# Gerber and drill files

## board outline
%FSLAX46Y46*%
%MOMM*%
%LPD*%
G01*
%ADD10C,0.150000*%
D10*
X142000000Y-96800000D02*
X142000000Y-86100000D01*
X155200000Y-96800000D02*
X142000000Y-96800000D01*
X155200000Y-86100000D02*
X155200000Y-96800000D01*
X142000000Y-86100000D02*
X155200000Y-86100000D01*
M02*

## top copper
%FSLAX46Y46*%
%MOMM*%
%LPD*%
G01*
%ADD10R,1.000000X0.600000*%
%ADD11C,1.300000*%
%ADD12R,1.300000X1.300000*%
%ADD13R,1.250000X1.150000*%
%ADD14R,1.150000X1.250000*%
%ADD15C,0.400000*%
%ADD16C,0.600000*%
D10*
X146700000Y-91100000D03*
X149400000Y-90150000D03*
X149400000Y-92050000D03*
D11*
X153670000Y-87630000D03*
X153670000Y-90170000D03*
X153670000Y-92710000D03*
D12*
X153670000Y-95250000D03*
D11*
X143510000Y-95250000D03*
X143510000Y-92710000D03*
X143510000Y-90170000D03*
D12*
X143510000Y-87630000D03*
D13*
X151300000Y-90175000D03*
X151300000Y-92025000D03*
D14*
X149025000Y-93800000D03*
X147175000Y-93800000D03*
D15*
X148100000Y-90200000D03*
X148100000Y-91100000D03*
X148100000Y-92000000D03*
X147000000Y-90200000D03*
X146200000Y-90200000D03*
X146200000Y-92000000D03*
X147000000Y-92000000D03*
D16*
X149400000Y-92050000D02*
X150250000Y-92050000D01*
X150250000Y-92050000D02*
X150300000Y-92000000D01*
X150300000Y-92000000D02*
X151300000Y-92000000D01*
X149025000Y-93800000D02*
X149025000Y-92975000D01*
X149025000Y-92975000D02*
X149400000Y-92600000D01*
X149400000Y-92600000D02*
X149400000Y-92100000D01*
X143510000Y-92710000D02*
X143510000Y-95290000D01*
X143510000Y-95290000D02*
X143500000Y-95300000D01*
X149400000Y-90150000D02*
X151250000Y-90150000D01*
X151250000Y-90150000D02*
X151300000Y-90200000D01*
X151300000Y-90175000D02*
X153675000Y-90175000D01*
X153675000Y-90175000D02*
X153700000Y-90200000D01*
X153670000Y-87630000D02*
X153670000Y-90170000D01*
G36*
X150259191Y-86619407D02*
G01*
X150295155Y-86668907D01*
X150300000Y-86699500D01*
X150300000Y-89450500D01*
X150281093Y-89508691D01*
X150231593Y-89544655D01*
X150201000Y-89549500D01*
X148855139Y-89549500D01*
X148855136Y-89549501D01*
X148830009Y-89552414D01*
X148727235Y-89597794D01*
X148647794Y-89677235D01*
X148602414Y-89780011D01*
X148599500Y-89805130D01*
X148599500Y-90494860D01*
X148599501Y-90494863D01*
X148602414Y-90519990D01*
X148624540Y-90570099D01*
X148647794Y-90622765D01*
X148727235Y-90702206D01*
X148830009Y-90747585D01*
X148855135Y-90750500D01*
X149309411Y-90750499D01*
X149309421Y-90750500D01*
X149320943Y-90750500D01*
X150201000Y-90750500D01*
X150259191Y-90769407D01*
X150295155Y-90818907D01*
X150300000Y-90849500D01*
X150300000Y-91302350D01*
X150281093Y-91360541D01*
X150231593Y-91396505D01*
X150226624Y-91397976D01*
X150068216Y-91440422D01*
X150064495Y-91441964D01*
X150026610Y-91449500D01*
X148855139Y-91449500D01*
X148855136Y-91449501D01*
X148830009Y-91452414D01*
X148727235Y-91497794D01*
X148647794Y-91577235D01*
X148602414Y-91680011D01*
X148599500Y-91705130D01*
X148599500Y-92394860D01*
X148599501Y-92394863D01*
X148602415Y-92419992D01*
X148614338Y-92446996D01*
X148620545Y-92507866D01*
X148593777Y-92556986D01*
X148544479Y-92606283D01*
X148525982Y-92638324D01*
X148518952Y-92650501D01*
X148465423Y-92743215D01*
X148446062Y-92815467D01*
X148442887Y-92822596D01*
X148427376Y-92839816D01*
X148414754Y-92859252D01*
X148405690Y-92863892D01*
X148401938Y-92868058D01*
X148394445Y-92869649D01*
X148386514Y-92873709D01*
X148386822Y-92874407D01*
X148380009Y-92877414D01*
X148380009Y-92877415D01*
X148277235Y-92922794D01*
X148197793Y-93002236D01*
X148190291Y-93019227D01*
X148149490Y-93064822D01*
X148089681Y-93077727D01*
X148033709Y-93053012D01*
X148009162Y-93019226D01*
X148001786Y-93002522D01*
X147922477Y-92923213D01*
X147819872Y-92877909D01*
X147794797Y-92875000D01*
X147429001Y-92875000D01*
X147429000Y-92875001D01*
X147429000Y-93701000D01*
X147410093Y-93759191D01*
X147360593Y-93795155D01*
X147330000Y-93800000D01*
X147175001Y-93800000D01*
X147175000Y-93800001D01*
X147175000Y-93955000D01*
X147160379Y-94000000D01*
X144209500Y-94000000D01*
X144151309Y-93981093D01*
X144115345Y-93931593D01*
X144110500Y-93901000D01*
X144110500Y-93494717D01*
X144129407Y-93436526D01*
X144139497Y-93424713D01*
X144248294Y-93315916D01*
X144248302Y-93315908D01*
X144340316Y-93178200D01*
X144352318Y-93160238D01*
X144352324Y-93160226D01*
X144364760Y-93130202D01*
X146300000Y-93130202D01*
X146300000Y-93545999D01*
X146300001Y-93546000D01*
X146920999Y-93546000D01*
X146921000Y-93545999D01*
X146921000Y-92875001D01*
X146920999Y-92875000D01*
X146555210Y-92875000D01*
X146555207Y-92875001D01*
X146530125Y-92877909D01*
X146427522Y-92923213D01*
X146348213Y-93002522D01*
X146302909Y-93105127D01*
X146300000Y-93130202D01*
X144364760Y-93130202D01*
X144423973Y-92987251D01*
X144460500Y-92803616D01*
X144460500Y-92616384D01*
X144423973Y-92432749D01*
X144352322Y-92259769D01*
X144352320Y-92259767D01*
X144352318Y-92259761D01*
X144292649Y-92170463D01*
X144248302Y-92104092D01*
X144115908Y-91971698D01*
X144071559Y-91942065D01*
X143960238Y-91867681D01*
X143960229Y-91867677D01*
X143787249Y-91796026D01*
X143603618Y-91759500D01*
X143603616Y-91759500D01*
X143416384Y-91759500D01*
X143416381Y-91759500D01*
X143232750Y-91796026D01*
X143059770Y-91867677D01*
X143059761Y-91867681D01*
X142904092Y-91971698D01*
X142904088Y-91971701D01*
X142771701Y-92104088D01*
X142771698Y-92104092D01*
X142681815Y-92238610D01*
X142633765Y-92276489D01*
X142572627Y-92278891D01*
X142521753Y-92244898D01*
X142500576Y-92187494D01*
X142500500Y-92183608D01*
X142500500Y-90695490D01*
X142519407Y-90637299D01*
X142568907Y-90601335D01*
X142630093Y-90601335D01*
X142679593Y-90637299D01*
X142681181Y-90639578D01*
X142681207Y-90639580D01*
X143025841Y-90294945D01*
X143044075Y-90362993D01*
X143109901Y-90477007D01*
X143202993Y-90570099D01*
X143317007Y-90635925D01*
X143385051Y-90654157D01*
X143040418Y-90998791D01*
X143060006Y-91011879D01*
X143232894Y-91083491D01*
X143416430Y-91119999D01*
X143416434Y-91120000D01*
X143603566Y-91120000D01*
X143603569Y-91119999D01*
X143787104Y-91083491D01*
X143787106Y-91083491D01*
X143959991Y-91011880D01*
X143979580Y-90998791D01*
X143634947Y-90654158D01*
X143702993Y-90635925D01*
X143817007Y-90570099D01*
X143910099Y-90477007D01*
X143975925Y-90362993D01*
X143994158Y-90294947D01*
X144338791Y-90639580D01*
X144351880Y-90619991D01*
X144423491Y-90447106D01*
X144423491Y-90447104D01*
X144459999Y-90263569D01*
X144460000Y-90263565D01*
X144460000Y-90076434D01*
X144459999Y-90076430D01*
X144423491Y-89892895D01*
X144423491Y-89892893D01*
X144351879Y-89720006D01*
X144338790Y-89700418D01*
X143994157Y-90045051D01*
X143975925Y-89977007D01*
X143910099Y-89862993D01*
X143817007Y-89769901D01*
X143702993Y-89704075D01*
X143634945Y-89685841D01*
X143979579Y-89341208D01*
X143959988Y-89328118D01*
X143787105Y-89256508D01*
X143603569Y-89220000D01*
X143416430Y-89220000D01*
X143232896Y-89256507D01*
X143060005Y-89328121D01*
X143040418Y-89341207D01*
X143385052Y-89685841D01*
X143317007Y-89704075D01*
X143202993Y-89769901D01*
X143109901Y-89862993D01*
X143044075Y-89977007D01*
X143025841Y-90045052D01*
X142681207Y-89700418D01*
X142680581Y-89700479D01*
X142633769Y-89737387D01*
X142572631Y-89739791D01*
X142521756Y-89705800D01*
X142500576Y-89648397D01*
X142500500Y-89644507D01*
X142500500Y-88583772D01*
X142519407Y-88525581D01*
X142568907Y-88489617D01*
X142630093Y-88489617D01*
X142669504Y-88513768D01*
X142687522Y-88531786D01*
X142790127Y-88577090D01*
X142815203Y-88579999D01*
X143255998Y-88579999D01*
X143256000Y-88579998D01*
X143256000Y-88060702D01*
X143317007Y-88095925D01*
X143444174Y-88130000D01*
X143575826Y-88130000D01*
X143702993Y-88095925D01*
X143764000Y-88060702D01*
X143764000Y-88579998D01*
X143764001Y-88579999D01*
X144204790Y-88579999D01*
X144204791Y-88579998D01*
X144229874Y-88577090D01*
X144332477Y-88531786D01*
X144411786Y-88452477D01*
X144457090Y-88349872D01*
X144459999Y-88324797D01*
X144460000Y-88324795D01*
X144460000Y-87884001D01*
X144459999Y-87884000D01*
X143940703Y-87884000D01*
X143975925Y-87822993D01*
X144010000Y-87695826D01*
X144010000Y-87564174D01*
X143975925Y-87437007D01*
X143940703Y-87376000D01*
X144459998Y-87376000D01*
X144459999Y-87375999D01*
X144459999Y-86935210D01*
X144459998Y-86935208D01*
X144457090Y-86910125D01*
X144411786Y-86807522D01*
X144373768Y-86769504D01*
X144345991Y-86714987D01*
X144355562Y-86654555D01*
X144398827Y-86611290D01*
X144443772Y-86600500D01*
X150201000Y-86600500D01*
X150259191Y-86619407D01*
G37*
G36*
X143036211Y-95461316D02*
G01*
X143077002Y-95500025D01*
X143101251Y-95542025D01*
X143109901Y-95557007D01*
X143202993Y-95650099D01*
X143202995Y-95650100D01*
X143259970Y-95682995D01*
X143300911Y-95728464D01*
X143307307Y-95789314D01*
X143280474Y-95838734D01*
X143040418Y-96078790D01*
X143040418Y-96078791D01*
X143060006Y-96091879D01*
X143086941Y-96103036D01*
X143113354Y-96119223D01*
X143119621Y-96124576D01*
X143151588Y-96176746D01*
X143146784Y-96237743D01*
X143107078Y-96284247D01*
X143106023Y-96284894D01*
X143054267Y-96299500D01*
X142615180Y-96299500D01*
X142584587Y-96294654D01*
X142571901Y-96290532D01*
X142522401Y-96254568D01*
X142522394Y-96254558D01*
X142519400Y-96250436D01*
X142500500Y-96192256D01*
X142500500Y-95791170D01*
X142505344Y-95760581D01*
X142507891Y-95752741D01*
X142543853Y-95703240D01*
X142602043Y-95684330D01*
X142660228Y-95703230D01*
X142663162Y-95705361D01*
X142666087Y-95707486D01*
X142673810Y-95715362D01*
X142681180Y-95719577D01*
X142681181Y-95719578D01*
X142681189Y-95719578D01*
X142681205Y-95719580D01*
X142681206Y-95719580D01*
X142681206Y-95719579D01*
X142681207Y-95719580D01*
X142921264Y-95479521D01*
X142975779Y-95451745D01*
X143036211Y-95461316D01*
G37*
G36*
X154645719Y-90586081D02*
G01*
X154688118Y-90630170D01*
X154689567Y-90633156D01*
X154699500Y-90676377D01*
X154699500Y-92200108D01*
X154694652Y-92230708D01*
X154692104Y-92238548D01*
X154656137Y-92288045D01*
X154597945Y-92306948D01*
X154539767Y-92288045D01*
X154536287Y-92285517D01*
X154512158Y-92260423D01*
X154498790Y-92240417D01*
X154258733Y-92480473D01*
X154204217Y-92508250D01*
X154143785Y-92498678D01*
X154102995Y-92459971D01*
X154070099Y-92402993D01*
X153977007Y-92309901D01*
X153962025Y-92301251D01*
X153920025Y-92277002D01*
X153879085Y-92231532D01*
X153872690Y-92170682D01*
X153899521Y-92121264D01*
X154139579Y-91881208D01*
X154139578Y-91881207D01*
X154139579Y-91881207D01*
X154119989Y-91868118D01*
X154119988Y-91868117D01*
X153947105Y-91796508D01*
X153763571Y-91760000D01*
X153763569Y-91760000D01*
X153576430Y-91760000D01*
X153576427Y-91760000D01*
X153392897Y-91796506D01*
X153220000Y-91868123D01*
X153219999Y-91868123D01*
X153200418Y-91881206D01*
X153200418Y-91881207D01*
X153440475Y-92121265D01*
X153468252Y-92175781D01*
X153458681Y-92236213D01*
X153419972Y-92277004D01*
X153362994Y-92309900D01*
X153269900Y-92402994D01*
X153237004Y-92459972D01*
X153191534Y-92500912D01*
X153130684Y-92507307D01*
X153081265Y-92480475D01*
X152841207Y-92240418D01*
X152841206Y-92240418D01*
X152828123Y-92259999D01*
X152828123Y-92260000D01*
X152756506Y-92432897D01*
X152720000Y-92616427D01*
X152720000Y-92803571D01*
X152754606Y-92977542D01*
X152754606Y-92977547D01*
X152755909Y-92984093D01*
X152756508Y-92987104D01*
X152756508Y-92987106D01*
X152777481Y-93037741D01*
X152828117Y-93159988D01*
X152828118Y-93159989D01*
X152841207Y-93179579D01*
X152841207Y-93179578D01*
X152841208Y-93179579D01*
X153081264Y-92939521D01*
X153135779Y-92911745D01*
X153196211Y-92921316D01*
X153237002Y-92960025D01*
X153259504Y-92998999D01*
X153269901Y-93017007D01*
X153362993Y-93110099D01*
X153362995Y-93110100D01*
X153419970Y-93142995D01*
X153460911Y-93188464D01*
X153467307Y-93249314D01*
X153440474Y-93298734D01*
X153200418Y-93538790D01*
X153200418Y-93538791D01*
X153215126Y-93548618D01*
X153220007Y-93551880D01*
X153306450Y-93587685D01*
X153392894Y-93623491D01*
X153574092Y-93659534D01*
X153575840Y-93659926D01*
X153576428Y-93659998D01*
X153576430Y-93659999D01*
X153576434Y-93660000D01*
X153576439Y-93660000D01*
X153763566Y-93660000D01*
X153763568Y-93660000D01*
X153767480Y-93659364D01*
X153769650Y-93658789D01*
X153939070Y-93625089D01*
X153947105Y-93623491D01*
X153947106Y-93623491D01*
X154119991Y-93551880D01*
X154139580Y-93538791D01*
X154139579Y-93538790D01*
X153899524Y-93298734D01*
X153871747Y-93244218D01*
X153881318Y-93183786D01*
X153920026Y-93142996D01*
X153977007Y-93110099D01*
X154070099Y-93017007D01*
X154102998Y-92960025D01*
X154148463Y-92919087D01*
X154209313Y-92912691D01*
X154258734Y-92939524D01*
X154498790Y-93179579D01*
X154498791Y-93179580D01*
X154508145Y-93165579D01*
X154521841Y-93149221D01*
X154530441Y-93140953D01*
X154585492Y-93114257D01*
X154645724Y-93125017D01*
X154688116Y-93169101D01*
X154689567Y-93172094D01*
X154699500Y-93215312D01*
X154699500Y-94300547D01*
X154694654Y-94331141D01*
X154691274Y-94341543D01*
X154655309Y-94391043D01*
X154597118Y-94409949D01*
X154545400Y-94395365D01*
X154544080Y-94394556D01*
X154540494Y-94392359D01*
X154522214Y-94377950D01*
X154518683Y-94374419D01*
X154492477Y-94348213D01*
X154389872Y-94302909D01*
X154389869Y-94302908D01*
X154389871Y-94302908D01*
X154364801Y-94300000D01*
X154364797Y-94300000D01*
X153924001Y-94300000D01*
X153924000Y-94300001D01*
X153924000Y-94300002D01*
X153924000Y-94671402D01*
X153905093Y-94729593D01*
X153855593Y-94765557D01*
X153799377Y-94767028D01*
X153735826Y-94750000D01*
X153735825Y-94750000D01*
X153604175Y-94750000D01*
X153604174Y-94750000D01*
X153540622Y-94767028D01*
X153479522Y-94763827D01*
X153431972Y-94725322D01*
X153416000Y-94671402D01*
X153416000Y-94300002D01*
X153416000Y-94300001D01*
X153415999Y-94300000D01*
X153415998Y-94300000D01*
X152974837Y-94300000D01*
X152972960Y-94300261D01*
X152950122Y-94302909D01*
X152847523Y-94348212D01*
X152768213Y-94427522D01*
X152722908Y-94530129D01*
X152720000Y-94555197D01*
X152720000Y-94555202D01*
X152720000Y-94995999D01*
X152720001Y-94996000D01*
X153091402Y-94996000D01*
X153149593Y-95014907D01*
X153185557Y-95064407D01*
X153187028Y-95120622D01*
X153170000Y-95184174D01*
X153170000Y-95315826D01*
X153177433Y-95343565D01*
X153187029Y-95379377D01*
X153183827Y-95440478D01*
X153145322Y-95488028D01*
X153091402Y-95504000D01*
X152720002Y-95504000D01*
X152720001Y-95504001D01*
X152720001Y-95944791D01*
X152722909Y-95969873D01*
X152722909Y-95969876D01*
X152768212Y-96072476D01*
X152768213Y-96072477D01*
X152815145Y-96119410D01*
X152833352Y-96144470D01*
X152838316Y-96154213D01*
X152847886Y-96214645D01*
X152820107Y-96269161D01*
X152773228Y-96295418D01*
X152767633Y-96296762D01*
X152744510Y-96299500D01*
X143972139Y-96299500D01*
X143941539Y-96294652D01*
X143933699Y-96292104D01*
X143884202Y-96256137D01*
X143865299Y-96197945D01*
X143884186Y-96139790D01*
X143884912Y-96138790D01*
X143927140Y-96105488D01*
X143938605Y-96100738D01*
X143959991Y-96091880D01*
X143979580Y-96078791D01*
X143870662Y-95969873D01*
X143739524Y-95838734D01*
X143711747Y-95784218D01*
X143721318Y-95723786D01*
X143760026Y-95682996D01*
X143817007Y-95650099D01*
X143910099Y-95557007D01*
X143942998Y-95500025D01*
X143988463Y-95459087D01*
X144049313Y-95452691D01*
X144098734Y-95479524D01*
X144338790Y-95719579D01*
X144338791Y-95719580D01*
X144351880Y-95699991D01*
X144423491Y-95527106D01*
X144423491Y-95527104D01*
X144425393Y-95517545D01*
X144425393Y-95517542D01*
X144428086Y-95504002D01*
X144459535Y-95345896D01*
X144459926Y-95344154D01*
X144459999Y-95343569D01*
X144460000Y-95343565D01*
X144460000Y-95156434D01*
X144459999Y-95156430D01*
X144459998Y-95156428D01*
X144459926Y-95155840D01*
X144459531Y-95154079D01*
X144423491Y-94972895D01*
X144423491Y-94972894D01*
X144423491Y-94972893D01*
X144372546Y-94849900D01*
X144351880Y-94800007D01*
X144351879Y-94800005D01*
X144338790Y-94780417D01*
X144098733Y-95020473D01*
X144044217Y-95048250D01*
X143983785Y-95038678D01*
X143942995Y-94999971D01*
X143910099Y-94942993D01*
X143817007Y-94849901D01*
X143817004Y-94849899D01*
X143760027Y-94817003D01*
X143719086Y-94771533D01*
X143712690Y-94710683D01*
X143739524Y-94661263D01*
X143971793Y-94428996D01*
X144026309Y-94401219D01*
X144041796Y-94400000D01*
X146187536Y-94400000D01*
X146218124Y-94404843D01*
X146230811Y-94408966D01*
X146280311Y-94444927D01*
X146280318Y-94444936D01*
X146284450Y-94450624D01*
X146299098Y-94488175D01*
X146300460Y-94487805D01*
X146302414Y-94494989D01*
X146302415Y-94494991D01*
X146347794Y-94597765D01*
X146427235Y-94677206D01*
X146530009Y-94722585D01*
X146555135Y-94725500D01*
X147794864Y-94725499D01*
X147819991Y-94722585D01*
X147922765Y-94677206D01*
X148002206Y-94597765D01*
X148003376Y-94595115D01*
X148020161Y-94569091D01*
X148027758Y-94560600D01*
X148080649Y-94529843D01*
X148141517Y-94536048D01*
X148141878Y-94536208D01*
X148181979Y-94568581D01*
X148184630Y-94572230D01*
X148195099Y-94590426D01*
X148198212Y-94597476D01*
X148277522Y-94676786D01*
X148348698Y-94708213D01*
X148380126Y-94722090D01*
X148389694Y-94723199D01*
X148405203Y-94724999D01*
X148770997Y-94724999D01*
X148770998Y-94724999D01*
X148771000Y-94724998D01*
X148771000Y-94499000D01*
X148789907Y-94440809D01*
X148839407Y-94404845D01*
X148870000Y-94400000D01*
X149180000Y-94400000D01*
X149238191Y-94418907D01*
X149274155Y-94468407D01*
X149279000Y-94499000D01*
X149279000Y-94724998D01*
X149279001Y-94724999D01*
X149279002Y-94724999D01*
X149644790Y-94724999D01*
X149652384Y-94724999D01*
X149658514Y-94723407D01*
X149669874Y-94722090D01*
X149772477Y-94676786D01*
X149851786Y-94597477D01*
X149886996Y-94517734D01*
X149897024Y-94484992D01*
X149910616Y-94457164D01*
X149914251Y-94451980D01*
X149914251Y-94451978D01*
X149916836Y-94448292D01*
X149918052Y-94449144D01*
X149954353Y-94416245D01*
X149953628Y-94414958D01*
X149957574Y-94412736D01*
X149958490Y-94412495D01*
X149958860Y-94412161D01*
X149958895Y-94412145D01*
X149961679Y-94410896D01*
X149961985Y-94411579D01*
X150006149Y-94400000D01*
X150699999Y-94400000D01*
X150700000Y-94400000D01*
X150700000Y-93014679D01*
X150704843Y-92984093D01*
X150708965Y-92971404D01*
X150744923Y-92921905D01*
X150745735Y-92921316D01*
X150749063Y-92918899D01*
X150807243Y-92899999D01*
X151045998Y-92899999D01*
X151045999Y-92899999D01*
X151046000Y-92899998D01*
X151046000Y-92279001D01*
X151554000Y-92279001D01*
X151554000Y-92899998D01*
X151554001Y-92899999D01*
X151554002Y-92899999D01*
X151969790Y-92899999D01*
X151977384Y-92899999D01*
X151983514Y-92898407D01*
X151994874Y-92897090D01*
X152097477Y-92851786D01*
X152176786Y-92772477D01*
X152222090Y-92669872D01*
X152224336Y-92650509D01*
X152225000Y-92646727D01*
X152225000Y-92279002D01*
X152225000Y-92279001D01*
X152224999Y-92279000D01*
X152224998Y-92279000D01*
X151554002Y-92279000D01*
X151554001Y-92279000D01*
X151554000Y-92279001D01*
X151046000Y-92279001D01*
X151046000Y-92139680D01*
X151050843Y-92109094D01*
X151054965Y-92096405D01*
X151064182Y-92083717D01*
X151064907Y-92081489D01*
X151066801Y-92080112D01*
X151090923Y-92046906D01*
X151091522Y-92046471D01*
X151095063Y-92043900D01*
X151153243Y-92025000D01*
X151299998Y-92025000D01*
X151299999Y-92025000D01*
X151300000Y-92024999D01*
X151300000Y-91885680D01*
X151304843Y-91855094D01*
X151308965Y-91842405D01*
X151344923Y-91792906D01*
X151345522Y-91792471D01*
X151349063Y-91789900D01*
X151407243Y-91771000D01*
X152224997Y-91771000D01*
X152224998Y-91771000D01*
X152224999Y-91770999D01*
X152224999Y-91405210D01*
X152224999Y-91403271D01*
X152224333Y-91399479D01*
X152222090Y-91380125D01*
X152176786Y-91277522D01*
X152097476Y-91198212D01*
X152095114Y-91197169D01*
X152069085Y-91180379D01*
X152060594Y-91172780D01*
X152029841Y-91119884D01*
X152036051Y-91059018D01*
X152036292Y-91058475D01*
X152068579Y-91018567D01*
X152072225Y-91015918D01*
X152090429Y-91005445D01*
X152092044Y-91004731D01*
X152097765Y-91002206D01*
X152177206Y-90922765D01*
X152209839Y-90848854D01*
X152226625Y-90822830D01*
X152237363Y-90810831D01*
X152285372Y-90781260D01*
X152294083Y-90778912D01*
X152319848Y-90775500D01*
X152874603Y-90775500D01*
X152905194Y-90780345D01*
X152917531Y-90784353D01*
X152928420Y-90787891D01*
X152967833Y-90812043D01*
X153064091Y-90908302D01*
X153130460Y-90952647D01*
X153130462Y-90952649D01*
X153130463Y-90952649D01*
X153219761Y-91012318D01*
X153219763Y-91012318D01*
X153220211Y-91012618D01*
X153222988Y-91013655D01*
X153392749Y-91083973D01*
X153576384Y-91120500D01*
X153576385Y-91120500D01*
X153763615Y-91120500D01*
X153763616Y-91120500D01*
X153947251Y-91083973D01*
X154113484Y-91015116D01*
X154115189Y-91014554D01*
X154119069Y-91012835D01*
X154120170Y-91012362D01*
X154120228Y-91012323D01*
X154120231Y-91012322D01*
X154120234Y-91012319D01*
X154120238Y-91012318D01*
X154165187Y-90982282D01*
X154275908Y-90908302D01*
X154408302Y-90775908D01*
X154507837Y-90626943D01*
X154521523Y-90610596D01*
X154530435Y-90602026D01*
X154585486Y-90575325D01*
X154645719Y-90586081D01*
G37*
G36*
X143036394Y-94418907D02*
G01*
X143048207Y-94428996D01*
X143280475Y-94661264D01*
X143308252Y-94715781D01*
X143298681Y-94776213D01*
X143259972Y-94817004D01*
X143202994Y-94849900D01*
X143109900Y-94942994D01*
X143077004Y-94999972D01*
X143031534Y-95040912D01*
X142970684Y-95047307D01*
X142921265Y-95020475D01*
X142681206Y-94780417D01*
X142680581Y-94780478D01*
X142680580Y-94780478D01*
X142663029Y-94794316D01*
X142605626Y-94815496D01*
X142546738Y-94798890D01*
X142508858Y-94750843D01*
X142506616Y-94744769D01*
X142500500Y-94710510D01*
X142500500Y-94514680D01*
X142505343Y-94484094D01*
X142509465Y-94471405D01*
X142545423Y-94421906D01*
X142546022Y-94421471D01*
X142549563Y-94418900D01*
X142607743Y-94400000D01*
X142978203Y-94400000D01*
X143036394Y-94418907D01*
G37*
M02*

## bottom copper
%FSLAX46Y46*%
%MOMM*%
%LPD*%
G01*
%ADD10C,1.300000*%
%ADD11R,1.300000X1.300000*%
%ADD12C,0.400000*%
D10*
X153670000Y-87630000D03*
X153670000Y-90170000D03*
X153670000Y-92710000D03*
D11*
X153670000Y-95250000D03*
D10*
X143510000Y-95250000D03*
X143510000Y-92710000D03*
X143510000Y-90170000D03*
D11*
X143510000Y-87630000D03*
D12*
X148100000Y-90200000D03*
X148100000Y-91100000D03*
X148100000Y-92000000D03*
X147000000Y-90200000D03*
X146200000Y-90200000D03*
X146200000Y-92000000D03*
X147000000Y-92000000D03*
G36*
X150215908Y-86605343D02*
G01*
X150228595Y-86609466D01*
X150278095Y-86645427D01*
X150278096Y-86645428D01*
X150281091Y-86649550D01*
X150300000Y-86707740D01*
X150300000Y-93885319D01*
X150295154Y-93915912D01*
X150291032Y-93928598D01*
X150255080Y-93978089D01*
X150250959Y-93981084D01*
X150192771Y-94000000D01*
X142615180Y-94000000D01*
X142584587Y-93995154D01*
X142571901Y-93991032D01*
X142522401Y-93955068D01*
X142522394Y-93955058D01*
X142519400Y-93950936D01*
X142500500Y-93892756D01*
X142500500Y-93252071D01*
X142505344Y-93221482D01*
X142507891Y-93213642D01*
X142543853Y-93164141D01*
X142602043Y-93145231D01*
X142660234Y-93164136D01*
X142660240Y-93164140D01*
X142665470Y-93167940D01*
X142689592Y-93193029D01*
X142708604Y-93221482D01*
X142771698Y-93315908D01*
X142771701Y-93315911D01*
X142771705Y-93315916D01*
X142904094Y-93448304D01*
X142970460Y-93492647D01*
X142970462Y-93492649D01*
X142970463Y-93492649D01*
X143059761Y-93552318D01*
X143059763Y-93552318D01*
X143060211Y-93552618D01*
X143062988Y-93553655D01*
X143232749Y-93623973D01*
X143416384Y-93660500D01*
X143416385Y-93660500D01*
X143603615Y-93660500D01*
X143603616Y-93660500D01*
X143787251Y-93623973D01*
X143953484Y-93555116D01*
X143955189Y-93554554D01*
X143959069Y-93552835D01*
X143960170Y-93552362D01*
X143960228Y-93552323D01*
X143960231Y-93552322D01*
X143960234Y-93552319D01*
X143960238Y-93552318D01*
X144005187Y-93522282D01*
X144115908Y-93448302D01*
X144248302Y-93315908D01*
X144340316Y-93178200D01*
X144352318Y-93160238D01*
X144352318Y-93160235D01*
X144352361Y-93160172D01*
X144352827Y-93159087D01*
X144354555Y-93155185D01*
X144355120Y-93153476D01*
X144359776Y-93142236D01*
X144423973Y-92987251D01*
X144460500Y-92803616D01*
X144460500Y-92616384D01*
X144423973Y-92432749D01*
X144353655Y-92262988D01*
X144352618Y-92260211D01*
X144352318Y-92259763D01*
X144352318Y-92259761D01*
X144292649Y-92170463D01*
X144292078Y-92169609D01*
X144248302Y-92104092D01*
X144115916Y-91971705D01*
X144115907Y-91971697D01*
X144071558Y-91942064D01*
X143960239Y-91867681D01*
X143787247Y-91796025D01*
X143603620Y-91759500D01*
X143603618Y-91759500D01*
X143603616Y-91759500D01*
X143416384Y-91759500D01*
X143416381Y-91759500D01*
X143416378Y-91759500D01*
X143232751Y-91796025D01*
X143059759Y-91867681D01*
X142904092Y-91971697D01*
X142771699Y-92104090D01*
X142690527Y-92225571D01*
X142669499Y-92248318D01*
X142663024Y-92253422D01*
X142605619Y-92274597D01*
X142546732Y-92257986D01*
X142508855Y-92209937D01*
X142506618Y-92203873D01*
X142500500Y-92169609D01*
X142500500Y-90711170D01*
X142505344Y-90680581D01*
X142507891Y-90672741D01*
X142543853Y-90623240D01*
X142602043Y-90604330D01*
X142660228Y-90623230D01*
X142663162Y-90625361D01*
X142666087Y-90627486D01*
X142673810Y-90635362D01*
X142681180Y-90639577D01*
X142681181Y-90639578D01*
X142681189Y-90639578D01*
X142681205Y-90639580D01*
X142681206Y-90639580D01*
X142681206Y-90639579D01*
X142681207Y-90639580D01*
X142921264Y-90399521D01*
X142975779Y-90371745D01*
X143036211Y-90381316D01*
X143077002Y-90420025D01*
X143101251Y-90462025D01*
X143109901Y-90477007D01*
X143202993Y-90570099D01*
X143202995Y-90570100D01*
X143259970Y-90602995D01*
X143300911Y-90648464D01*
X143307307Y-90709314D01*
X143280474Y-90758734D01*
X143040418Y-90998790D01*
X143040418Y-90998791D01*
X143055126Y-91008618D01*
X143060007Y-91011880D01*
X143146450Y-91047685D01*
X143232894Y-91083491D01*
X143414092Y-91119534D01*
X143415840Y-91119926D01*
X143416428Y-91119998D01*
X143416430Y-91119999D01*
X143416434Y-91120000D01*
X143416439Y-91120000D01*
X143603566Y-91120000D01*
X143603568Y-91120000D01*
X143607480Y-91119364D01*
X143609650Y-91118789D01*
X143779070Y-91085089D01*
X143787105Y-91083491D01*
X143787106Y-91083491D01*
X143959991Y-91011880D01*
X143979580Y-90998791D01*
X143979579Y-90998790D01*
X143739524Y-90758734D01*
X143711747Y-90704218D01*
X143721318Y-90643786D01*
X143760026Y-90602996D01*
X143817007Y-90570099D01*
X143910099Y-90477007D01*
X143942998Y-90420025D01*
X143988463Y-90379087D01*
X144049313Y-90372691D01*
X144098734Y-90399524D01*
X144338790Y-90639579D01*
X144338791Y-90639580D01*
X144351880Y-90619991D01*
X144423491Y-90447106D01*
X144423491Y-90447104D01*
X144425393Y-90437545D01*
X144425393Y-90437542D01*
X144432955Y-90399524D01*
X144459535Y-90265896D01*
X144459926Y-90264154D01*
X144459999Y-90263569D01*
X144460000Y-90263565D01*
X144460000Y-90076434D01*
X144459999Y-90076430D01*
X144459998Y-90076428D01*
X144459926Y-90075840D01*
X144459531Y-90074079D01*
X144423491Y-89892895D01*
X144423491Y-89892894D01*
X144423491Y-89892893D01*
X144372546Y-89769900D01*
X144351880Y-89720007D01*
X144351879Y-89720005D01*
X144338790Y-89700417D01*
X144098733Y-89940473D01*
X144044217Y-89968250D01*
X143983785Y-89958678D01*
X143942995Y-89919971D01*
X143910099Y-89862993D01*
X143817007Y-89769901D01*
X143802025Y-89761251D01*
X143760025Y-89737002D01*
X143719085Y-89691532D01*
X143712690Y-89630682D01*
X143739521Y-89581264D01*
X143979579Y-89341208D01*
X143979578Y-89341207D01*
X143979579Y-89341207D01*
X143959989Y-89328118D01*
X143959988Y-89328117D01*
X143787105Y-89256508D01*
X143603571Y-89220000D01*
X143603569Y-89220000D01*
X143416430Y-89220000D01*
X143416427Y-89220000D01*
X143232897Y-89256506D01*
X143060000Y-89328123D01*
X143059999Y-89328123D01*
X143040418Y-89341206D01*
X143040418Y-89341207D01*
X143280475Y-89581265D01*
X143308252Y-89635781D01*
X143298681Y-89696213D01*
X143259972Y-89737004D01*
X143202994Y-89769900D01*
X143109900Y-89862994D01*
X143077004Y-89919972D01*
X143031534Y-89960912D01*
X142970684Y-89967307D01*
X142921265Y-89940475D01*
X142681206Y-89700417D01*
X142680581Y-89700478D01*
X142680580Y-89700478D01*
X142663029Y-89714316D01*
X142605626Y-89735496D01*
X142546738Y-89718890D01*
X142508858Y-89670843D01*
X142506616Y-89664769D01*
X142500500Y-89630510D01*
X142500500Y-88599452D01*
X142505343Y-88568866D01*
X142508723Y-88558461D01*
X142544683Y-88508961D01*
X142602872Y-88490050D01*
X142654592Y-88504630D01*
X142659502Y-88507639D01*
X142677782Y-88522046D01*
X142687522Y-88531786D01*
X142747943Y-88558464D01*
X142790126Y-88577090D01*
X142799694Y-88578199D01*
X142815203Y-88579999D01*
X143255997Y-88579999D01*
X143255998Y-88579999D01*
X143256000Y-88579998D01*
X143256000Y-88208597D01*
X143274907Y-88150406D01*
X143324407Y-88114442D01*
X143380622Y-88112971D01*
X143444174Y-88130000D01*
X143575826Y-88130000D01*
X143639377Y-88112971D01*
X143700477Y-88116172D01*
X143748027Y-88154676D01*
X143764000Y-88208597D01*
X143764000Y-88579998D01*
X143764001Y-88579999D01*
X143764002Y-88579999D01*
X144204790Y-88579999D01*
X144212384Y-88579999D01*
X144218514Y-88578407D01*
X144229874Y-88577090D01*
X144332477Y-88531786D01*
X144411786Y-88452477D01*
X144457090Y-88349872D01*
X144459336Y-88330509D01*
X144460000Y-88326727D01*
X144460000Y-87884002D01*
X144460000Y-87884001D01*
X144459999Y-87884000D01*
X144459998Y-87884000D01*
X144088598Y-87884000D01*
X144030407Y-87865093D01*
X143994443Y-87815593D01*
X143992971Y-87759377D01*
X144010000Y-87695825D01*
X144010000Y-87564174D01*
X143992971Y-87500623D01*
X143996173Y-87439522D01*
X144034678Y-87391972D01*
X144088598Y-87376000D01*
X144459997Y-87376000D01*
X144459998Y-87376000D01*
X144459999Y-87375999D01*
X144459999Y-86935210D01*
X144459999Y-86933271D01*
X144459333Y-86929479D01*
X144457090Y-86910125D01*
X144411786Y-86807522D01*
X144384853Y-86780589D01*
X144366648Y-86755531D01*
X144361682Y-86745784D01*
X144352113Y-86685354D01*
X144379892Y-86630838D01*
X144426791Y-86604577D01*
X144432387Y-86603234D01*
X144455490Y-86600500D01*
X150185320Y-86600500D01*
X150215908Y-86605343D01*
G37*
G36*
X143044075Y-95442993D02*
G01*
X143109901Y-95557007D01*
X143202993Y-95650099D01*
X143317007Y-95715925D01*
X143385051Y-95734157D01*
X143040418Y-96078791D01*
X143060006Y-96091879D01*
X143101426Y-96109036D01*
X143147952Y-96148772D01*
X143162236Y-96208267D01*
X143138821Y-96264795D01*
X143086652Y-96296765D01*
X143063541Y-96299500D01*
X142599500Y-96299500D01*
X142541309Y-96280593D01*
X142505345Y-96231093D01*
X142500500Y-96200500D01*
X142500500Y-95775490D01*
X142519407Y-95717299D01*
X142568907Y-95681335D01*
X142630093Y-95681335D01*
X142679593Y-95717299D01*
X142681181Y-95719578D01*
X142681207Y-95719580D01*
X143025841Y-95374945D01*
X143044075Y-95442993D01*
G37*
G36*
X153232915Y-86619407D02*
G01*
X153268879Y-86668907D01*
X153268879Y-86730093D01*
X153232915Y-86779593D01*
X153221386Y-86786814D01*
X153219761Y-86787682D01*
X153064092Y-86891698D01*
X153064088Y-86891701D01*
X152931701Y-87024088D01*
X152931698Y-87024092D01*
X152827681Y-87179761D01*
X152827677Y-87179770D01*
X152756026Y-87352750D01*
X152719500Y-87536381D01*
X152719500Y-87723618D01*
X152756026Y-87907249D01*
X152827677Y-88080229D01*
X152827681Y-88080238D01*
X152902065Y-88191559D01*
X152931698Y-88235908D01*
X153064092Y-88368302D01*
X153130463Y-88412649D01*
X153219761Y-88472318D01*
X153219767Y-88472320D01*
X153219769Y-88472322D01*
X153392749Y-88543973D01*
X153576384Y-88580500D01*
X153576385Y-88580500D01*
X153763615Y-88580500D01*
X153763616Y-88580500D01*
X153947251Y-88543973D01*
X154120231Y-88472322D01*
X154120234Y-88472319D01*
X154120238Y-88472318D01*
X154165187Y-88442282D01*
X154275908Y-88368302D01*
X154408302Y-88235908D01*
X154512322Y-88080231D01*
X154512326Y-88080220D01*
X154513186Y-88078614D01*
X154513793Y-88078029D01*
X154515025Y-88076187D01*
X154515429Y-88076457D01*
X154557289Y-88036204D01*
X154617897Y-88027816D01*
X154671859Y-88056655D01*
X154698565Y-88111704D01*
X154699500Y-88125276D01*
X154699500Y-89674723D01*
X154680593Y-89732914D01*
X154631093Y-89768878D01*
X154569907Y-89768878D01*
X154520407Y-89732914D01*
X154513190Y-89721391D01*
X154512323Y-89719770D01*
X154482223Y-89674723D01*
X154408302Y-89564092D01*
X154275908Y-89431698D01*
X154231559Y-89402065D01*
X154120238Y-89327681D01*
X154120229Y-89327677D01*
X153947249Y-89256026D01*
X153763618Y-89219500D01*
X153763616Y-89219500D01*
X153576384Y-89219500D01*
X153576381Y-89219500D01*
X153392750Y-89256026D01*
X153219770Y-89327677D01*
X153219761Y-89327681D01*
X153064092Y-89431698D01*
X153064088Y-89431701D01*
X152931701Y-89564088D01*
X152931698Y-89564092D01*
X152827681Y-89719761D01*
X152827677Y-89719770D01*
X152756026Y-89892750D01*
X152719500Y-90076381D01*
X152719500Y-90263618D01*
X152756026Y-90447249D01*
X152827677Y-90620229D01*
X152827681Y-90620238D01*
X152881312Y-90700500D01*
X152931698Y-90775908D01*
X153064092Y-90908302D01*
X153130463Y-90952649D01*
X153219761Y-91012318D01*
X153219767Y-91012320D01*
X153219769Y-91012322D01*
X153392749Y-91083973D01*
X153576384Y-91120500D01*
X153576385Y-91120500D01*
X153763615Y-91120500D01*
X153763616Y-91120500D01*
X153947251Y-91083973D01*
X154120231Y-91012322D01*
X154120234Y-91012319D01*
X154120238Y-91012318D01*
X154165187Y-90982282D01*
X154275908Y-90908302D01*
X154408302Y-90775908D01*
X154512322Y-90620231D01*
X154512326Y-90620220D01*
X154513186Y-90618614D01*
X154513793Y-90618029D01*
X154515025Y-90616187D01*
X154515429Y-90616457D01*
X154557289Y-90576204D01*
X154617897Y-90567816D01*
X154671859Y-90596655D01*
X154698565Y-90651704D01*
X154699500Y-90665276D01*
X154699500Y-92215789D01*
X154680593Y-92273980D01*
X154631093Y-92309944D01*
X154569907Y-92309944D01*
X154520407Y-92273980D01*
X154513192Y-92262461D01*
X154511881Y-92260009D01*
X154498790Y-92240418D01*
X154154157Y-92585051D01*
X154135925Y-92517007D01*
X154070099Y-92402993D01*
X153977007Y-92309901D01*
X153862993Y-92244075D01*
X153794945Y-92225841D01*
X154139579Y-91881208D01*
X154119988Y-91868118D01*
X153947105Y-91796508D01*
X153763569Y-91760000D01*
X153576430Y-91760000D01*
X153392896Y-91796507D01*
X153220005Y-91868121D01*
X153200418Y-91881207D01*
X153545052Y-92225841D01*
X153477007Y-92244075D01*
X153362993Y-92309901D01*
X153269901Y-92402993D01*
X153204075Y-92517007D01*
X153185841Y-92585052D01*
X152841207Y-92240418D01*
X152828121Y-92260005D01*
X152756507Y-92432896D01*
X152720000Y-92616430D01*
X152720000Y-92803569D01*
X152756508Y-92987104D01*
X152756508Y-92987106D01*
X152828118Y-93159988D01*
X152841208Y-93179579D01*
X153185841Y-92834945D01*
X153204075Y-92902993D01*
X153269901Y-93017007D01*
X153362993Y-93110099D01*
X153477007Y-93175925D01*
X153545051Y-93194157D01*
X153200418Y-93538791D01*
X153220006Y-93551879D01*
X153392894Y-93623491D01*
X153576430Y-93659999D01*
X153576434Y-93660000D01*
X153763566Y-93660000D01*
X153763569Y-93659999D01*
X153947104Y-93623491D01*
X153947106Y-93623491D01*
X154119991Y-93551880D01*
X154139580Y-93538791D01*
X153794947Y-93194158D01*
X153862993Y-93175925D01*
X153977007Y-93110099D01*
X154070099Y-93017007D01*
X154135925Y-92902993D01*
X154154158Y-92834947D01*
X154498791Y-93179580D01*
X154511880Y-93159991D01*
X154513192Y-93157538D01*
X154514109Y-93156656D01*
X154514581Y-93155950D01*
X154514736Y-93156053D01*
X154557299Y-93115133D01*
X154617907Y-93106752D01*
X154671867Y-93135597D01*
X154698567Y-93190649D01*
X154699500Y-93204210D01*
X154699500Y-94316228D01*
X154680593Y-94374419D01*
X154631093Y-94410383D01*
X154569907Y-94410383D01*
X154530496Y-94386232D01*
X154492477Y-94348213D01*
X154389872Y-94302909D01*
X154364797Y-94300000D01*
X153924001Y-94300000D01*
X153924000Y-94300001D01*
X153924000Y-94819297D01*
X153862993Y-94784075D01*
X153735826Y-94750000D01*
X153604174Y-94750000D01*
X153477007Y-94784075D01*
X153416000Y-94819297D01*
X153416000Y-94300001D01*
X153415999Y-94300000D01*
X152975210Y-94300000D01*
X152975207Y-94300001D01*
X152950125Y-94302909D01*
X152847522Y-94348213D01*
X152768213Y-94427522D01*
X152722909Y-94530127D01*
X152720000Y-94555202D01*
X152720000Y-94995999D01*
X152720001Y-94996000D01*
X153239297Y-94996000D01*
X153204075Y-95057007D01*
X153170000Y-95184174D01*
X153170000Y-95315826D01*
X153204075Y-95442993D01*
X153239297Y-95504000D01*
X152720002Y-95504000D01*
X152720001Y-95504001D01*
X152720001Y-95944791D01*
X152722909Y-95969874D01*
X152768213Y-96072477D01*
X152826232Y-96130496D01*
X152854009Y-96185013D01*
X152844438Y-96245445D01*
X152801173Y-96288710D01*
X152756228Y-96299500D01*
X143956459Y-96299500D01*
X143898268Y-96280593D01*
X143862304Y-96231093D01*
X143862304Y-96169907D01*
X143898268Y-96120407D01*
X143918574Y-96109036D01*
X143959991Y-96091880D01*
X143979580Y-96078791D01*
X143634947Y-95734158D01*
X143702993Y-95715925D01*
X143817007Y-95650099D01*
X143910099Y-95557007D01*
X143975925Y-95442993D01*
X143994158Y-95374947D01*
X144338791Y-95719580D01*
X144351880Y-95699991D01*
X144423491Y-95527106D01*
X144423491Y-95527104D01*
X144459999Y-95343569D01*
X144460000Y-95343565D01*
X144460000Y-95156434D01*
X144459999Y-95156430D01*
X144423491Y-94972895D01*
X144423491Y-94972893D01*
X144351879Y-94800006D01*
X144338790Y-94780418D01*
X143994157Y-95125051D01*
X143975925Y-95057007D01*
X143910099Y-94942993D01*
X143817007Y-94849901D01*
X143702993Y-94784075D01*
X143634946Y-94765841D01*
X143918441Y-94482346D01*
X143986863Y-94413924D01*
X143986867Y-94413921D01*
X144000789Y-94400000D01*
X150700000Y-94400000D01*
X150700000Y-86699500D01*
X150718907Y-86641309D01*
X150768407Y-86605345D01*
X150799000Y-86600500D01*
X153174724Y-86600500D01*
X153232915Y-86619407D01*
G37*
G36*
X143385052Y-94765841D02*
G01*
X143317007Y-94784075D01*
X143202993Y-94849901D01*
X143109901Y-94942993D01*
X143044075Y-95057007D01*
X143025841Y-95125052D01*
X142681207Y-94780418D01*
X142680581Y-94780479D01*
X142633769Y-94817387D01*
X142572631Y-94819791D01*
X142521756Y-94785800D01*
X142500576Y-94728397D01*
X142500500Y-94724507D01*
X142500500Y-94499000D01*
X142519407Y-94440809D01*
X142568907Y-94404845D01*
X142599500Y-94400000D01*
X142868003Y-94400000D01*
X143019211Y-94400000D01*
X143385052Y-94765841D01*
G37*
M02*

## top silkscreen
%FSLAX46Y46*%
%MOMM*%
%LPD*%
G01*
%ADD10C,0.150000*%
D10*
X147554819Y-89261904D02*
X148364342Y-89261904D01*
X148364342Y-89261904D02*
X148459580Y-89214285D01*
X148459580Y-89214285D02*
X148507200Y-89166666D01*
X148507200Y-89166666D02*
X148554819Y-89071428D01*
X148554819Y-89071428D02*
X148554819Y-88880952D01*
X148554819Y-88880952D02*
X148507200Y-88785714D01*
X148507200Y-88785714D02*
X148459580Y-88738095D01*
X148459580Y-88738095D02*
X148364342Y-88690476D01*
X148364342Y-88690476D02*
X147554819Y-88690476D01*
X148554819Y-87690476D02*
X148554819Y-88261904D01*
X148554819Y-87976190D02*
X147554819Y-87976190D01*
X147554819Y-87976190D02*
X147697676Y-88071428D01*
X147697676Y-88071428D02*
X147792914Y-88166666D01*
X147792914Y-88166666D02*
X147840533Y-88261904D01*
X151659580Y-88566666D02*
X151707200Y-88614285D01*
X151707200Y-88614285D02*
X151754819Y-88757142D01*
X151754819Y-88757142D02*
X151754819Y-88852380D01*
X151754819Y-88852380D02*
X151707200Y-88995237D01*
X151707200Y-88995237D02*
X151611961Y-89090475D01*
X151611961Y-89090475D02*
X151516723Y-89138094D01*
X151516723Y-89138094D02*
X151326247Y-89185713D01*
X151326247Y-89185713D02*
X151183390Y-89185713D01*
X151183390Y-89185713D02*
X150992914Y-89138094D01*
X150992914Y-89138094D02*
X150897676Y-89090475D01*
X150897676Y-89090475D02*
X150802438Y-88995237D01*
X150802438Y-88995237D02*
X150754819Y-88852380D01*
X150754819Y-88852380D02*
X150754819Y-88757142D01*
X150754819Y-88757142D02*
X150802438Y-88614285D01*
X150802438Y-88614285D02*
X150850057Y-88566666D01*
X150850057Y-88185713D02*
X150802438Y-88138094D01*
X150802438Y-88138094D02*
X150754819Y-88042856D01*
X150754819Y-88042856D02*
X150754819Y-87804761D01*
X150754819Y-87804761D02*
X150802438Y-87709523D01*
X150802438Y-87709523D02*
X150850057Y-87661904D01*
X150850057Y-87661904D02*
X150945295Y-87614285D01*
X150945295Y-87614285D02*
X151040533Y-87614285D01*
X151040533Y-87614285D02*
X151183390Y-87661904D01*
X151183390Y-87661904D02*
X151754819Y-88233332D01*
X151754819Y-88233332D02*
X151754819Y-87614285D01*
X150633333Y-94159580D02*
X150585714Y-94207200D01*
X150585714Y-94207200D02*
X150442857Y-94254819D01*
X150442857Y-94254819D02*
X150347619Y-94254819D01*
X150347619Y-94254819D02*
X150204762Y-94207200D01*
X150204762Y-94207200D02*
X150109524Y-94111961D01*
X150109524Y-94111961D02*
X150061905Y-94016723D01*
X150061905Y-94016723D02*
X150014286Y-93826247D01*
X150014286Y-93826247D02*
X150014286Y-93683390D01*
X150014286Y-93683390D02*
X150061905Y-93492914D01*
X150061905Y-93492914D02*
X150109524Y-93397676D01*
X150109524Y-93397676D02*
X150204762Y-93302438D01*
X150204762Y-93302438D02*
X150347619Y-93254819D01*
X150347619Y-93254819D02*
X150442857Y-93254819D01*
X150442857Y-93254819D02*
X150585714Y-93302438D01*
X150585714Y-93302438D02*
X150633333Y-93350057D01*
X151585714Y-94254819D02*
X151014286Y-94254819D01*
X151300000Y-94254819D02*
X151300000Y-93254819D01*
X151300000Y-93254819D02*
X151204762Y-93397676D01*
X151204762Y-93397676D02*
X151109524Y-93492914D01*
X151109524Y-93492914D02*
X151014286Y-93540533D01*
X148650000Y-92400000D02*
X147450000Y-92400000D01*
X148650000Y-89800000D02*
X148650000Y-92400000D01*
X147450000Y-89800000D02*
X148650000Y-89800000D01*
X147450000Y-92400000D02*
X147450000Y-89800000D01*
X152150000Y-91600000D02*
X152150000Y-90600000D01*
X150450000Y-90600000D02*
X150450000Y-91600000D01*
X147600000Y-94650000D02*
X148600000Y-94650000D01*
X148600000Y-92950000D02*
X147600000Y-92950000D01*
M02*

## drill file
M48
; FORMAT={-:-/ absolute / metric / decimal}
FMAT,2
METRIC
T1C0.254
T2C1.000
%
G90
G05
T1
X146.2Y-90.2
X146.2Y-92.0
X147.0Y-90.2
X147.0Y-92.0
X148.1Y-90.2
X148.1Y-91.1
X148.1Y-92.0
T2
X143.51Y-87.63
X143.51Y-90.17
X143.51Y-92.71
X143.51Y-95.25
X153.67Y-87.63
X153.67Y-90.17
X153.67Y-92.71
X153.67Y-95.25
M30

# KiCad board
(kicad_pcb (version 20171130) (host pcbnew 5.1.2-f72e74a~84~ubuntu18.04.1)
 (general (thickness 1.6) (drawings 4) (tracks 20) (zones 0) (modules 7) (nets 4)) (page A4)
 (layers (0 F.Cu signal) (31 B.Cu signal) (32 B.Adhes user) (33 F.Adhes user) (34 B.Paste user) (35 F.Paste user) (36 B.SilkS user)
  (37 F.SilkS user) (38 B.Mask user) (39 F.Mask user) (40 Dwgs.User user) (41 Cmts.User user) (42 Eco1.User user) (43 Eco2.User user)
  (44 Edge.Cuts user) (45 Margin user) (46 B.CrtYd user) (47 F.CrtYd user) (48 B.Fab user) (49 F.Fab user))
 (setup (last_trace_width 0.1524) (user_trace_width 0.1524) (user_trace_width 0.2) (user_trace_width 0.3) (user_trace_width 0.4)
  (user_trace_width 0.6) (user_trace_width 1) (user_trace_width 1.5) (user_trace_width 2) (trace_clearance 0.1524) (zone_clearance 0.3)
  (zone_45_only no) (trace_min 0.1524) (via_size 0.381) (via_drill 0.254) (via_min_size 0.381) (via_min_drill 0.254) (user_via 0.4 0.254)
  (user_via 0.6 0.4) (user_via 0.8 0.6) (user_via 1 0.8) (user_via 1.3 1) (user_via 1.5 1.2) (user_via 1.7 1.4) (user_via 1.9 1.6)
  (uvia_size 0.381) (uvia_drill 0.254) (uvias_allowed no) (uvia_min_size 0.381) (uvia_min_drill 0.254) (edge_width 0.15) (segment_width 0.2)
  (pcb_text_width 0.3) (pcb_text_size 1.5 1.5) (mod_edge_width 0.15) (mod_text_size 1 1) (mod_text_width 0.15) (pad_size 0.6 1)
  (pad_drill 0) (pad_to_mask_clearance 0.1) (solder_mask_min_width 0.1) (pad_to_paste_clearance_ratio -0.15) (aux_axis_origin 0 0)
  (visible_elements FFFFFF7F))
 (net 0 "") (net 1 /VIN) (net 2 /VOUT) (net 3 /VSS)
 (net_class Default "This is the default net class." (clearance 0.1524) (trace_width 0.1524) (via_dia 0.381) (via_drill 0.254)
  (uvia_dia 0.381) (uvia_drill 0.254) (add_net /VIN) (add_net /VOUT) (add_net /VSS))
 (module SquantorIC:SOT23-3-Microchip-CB (layer F.Cu) (at 148.05 91.1 90)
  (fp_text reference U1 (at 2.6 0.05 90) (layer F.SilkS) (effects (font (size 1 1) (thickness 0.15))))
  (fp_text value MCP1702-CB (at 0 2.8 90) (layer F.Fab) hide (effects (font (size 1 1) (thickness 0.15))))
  (fp_line (start -1.3 0.6) (end -1.3 -0.6) (layer F.SilkS) (width 0.15))
  (fp_line (start 1.3 0.6) (end -1.3 0.6) (layer F.SilkS) (width 0.15))
  (fp_line (start 1.3 -0.6) (end 1.3 0.6) (layer F.SilkS) (width 0.15))
  (fp_line (start -1.3 -0.6) (end 1.3 -0.6) (layer F.SilkS) (width 0.15))
  (pad 3 smd rect (at 0 -1.35 90) (size 0.6 1) (layers F.Cu F.Paste F.Mask) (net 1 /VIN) (zone_connect 2))
  (pad 2 smd rect (at 0.95 1.35 90) (size 0.6 1) (layers F.Cu F.Paste F.Mask) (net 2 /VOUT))
  (pad 1 smd rect (at -0.95 1.35 90) (size 0.6 1) (layers F.Cu F.Paste F.Mask) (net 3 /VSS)))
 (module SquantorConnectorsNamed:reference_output (layer B.Cu) (at 153.67 91.44 90)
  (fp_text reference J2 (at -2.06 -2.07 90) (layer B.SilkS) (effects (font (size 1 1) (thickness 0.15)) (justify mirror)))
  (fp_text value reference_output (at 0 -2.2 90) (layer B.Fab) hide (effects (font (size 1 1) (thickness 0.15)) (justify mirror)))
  (pad 4 thru_hole circle (at 3.81 0 270) (size 1.3 1.3) (drill 1) (layers *.Cu *.Mask) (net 2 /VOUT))
  (pad 3 thru_hole circle (at 1.27 0 270) (size 1.3 1.3) (drill 1) (layers *.Cu *.Mask) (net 2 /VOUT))
  (pad 2 thru_hole circle (at -1.27 0 270) (size 1.3 1.3) (drill 1) (layers *.Cu *.Mask) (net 3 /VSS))
  (pad 1 thru_hole rect (at -3.81 0 270) (size 1.3 1.3) (drill 1) (layers *.Cu *.Mask) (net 3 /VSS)))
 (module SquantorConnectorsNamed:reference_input (layer B.Cu) (at 143.51 91.44 270)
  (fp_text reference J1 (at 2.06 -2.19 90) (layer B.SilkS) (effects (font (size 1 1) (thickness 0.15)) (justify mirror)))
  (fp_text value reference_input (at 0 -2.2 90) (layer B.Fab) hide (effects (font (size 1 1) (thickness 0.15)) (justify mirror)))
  (pad 4 thru_hole circle (at 3.81 0 90) (size 1.3 1.3) (drill 1) (layers *.Cu *.Mask) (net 3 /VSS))
  (pad 3 thru_hole circle (at 1.27 0 90) (size 1.3 1.3) (drill 1) (layers *.Cu *.Mask) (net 3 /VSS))
  (pad 2 thru_hole circle (at -1.27 0 90) (size 1.3 1.3) (drill 1) (layers *.Cu *.Mask) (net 1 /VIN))
  (pad 1 thru_hole rect (at -3.81 0 90) (size 1.3 1.3) (drill 1) (layers *.Cu *.Mask) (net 1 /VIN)))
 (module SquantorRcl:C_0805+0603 (layer F.Cu) (at 151.3 91.1 270)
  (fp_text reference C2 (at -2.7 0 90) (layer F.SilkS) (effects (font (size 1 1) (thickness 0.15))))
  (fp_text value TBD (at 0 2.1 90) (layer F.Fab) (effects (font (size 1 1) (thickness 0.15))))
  (fp_line (start 0.5 -0.85) (end -0.5 -0.85) (layer F.SilkS) (width 0.15))
  (fp_line (start -0.5 0.85) (end 0.5 0.85) (layer F.SilkS) (width 0.15))
  (pad 1 smd rect (at -0.925 0 270) (size 1.15 1.25) (layers F.Cu F.Paste F.Mask) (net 2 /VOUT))
  (pad 2 smd rect (at 0.925 0 270) (size 1.15 1.25) (layers F.Cu F.Paste F.Mask) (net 3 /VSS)))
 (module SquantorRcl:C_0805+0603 (layer F.Cu) (at 148.1 93.8 180)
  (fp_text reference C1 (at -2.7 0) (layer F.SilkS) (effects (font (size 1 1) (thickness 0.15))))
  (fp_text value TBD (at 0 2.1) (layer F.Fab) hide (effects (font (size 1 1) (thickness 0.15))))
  (fp_line (start 0.5 -0.85) (end -0.5 -0.85) (layer F.SilkS) (width 0.15))
  (fp_line (start -0.5 0.85) (end 0.5 0.85) (layer F.SilkS) (width 0.15))
  (pad 1 smd rect (at -0.925 0 180) (size 1.15 1.25) (layers F.Cu F.Paste F.Mask) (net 3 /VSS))
  (pad 2 smd rect (at 0.925 0 180) (size 1.15 1.25) (layers F.Cu F.Paste F.Mask) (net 1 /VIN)))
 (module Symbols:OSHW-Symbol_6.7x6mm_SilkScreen (layer B.Cu) (at 148.6 90 180)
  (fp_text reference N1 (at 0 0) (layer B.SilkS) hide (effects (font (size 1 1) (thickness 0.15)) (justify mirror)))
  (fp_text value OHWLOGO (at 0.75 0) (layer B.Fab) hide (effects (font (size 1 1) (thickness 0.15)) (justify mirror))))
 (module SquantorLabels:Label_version (layer F.Cu) (at 149.3 96.1)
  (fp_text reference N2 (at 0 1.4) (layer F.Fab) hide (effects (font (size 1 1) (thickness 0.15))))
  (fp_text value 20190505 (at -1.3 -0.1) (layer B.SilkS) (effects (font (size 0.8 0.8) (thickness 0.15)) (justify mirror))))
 (gr_line (start 142 96.8) (end 142 86.1) (layer Edge.Cuts) (width 0.15))
 (gr_line (start 155.2 96.8) (end 142 96.8) (layer Edge.Cuts) (width 0.15))
 (gr_line (start 155.2 86.1) (end 155.2 96.8) (layer Edge.Cuts) (width 0.15))
 (gr_line (start 142 86.1) (end 155.2 86.1) (layer Edge.Cuts) (width 0.15))
 (segment (start 149.4 92.05) (end 150.25 92.05) (width 0.6) (layer F.Cu) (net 3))
 (segment (start 150.25 92.05) (end 150.3 92) (width 0.6) (layer F.Cu) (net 3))
 (segment (start 150.3 92) (end 151.3 92) (width 0.6) (layer F.Cu) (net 3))
 (segment (start 149.025 93.8) (end 149.025 92.975) (width 0.6) (layer F.Cu) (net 3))
 (segment (start 149.025 92.975) (end 149.4 92.6) (width 0.6) (layer F.Cu) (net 3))
 (segment (start 149.4 92.6) (end 149.4 92.1) (width 0.6) (layer F.Cu) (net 3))
 (segment (start 143.51 92.71) (end 143.51 95.29) (width 0.6) (layer F.Cu) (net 3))
 (segment (start 143.51 95.29) (end 143.5 95.3) (width 0.6) (layer F.Cu) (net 3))
 (via (at 148.1 90.2) (size 0.4) (drill 0.254) (layers F.Cu B.Cu) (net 1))
 (via (at 148.1 91.1) (size 0.4) (drill 0.254) (layers F.Cu B.Cu) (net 1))
 (via (at 148.1 92) (size 0.4) (drill 0.254) (layers F.Cu B.Cu) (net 1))
 (via (at 147 90.2) (size 0.4) (drill 0.254) (layers F.Cu B.Cu) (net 1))
 (via (at 146.2 90.2) (size 0.4) (drill 0.254) (layers F.Cu B.Cu) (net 1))
 (via (at 146.2 92) (size 0.4) (drill 0.254) (layers F.Cu B.Cu) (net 1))
 (via (at 147 92) (size 0.4) (drill 0.254) (layers F.Cu B.Cu) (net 1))
 (segment (start 149.4 90.15) (end 151.25 90.15) (width 0.6) (layer F.Cu) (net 2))
 (segment (start 151.25 90.15) (end 151.3 90.2) (width 0.6) (layer F.Cu) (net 2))
 (segment (start 151.3 90.175) (end 153.675 90.175) (width 0.6) (layer F.Cu) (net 2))
 (segment (start 153.675 90.175) (end 153.7 90.2) (width 0.6) (layer F.Cu) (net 2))
 (segment (start 153.67 87.63) (end 153.67 90.17) (width 0.6) (layer F.Cu) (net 2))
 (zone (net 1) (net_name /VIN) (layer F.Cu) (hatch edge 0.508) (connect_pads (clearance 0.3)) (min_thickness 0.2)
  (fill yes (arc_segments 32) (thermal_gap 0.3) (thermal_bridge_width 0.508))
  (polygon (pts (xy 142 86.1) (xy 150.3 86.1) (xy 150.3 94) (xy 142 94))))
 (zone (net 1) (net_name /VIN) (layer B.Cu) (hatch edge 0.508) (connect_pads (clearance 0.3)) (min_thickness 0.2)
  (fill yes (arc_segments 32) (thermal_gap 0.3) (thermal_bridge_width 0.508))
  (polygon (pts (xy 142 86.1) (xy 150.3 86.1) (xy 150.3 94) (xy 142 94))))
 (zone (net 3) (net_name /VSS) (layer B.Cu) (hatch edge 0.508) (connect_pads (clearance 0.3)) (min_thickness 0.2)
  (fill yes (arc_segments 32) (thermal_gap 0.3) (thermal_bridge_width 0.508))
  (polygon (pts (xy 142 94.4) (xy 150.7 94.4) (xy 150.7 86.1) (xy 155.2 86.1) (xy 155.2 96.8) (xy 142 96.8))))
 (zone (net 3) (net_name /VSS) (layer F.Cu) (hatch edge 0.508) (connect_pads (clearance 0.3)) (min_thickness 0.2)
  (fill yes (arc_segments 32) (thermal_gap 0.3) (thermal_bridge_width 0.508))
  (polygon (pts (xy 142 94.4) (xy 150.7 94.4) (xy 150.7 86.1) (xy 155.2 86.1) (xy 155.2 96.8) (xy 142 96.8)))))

